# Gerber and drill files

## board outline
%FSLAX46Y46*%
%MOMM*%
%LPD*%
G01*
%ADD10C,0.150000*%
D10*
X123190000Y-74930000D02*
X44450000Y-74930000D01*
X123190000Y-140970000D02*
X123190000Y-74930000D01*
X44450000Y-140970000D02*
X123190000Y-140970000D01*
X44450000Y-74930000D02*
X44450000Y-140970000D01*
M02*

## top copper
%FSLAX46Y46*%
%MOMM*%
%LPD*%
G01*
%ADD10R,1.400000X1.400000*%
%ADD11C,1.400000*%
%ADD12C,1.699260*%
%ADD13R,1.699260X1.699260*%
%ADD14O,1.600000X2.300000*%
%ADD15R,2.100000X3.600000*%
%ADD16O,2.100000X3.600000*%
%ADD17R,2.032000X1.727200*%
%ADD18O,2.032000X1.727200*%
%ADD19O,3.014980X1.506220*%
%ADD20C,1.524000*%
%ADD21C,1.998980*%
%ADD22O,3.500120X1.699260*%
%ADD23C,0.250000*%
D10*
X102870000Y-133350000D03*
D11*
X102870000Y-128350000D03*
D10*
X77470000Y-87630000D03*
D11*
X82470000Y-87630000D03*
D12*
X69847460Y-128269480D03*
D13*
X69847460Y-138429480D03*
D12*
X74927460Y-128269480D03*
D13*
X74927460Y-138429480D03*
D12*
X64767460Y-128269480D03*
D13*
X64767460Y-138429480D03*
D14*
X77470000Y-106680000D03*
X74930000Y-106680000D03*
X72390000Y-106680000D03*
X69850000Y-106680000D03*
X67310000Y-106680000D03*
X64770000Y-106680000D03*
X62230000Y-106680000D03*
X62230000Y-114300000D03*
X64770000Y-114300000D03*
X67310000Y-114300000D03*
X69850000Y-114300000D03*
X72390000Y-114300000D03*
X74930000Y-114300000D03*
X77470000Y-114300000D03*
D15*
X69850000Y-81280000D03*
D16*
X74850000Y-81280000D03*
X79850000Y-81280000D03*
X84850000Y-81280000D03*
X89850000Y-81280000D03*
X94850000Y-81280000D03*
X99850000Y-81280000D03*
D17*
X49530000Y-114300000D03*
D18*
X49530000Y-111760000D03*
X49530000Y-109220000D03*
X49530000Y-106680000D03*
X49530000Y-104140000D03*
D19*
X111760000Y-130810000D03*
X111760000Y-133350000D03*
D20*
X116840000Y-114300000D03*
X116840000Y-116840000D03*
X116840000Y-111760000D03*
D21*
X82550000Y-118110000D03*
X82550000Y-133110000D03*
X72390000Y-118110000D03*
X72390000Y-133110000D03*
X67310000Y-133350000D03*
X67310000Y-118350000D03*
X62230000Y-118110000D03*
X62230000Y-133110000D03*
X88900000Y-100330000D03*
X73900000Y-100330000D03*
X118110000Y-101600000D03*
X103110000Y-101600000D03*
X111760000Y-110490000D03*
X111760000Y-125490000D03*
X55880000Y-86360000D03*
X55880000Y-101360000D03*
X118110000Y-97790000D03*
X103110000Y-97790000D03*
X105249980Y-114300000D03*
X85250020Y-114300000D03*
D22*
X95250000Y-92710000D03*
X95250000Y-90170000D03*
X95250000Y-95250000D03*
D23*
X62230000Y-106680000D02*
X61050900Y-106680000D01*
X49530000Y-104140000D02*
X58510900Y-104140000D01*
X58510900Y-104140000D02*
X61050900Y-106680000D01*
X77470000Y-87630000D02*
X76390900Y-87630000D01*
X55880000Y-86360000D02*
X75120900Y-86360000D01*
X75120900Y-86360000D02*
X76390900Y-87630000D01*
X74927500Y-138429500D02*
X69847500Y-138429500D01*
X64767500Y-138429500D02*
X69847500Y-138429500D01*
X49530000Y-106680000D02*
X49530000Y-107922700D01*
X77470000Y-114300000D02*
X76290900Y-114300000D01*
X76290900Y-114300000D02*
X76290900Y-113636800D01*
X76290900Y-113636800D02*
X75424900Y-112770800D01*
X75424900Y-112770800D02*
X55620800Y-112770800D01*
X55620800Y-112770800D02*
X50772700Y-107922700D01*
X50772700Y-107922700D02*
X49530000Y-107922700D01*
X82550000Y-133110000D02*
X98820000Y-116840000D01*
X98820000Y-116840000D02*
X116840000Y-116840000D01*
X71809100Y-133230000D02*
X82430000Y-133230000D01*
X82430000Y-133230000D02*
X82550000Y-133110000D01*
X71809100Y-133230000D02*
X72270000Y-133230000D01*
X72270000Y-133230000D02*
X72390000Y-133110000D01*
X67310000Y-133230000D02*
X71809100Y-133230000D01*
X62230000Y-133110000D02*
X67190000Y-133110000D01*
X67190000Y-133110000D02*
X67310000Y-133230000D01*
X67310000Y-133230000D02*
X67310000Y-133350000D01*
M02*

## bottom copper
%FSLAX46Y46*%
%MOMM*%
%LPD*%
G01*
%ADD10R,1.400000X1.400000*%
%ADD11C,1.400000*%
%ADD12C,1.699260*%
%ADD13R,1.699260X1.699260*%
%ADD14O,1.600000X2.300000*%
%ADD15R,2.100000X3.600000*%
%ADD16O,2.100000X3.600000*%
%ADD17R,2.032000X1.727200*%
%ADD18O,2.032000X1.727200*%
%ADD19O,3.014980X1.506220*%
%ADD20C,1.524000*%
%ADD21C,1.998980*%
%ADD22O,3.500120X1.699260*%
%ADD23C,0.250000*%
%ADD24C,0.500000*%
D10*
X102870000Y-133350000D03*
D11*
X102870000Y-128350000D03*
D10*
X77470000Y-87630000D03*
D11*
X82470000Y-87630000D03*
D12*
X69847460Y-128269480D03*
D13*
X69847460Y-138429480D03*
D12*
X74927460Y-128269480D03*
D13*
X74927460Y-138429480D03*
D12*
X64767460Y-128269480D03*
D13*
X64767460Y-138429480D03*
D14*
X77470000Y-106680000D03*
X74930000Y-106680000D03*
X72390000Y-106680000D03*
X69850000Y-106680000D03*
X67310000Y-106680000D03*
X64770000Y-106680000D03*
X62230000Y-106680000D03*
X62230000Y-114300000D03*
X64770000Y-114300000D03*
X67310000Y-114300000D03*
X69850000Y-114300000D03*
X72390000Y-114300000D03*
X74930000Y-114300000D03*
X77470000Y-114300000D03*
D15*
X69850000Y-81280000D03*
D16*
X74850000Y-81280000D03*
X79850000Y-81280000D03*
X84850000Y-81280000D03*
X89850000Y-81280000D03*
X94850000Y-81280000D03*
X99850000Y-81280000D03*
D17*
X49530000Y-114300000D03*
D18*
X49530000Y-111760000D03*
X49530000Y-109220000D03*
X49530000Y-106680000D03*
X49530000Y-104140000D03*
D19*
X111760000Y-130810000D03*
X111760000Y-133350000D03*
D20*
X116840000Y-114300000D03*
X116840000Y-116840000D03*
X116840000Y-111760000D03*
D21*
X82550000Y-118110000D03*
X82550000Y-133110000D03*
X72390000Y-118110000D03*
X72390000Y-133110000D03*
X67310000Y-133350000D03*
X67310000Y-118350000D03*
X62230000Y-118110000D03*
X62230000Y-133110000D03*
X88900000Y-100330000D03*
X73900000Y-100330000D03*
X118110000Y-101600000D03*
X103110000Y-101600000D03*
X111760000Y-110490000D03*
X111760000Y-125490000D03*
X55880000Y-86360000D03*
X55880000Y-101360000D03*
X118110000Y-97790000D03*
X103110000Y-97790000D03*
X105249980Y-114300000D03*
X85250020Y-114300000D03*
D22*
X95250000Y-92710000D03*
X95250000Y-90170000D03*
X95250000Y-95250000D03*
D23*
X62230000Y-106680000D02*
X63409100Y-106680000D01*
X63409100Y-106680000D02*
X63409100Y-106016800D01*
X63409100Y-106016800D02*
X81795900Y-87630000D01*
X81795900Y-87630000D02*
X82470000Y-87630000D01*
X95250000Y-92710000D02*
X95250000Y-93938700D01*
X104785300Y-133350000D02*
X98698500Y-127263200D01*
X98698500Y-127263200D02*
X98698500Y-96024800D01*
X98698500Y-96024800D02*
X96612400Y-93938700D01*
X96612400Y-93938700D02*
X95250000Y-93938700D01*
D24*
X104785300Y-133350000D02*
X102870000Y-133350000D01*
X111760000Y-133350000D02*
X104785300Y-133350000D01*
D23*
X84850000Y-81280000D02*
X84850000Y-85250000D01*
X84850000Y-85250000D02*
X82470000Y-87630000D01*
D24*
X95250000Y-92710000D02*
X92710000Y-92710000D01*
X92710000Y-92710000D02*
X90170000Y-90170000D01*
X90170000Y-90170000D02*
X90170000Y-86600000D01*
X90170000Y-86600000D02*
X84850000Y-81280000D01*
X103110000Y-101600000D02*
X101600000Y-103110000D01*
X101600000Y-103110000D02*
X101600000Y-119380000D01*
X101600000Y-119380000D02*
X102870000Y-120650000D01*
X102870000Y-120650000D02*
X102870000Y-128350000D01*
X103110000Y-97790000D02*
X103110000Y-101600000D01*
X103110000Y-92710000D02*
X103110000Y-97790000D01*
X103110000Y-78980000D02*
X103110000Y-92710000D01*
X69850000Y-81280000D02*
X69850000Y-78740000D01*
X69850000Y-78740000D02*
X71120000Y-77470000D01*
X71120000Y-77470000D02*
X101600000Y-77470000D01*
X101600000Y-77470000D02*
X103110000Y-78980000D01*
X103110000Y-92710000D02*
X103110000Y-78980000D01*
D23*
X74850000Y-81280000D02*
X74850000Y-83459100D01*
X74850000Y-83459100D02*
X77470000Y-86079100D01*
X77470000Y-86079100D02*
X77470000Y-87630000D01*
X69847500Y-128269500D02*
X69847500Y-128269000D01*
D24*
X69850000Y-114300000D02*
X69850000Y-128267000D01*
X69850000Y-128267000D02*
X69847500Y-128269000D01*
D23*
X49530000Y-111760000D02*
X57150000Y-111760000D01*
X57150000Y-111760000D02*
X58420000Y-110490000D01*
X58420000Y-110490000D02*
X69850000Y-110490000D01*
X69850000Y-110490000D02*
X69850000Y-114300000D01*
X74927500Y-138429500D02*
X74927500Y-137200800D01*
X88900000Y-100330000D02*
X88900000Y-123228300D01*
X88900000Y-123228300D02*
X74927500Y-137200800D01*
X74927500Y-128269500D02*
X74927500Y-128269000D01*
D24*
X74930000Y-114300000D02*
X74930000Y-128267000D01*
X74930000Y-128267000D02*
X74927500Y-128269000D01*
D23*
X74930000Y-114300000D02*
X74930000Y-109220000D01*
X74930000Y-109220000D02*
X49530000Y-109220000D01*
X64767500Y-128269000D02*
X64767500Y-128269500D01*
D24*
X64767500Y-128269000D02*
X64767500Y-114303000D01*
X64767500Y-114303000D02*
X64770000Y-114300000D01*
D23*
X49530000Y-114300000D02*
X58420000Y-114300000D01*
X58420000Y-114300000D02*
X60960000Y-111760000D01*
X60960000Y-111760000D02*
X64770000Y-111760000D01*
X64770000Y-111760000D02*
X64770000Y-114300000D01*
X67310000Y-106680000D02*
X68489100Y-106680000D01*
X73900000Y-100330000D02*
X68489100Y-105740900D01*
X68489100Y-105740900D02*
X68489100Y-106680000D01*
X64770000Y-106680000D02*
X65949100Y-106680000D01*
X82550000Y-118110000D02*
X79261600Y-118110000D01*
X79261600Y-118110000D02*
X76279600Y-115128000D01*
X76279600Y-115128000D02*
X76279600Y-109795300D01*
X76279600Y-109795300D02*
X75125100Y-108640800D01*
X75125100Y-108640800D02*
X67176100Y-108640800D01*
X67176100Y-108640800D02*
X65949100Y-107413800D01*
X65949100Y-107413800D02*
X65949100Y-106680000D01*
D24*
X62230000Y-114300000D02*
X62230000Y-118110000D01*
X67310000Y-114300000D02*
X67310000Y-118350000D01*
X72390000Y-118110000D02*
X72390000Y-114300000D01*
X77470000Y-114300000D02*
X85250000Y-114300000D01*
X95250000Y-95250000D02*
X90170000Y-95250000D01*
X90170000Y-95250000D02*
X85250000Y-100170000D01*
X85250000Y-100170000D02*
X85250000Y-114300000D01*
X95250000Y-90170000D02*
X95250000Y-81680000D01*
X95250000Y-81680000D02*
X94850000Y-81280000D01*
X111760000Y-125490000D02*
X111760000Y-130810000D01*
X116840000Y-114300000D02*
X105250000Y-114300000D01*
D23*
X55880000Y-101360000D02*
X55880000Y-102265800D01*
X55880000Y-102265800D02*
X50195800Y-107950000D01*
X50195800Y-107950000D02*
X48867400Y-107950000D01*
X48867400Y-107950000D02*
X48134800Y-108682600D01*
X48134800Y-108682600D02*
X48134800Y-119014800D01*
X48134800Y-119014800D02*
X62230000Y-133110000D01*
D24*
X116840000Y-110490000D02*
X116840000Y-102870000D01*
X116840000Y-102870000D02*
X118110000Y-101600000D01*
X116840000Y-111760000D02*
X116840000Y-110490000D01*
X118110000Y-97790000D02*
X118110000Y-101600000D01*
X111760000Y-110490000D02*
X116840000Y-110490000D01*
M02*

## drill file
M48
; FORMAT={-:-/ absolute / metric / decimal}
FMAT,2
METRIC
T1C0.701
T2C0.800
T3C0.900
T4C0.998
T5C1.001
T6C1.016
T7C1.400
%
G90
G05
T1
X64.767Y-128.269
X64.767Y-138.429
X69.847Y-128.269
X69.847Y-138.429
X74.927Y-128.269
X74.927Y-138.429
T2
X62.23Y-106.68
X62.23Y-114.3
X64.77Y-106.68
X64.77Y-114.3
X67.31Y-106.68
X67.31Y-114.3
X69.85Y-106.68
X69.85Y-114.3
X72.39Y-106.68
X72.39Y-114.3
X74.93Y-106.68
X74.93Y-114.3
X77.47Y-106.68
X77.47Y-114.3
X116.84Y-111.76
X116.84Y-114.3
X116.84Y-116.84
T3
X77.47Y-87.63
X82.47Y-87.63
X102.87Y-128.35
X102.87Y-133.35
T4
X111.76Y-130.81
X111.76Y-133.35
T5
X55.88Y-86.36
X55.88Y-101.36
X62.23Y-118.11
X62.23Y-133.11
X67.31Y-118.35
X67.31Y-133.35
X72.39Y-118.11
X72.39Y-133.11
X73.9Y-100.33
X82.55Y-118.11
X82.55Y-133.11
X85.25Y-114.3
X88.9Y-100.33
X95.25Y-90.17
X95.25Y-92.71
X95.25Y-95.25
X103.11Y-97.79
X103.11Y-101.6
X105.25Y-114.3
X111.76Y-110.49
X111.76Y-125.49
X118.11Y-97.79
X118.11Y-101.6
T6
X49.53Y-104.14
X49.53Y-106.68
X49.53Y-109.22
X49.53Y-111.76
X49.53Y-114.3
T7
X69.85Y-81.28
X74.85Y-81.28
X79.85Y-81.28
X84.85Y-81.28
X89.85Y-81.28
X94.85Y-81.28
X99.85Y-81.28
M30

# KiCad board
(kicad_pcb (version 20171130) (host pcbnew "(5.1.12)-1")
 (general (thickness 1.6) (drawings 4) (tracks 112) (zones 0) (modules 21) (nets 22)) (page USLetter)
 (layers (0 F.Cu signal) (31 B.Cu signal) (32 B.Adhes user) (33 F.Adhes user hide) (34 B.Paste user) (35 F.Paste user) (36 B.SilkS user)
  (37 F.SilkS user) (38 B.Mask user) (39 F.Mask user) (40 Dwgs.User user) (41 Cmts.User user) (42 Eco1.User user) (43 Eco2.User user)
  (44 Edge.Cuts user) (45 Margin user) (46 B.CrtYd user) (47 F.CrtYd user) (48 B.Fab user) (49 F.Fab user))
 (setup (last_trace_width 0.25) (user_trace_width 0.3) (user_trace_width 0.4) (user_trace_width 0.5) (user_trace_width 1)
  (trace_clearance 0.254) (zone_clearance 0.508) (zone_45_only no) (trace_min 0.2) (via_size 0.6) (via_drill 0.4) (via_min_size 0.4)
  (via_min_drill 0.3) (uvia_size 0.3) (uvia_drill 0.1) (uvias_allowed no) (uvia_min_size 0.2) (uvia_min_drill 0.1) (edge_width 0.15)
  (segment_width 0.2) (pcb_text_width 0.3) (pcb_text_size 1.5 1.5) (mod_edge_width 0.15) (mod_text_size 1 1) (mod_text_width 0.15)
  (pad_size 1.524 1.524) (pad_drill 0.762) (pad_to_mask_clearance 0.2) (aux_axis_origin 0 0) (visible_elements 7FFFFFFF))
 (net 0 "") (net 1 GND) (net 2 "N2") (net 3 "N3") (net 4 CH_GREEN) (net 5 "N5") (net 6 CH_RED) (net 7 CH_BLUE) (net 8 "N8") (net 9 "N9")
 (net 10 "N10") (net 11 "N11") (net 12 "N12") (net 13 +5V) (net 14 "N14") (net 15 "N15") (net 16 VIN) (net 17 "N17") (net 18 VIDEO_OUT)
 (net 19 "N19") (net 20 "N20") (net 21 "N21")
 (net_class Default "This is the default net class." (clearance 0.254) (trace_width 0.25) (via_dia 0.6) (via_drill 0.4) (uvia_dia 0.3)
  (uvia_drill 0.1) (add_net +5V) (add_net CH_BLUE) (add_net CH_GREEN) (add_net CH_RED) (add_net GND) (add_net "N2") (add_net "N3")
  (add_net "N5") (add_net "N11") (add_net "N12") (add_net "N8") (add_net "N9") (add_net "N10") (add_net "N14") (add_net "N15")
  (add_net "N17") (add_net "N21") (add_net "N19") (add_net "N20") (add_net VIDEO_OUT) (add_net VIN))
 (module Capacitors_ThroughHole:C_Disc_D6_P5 (layer F.Cu) (at 102.87 133.35 90)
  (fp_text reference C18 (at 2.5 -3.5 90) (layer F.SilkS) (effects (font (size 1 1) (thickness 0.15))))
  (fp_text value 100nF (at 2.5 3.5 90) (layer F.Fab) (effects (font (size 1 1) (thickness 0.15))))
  (pad 1 thru_hole rect (at 0 0 90) (size 1.4 1.4) (drill 0.9) (layers *.Cu *.Mask F.SilkS) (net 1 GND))
  (pad 2 thru_hole circle (at 5 0 90) (size 1.4 1.4) (drill 0.9) (layers *.Cu *.Mask F.SilkS) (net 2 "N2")))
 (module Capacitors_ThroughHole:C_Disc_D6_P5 (layer F.Cu) (at 77.47 87.63)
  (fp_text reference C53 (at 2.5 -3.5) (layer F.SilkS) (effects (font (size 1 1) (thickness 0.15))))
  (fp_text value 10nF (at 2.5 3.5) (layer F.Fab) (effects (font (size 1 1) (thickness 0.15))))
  (pad 1 thru_hole rect (at 0 0) (size 1.4 1.4) (drill 0.9) (layers *.Cu *.Mask F.SilkS) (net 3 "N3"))
  (pad 2 thru_hole circle (at 5 0) (size 1.4 1.4) (drill 0.9) (layers *.Cu *.Mask F.SilkS) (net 1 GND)))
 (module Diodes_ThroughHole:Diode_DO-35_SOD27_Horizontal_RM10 (layer F.Cu) (at 69.85 138.43 90)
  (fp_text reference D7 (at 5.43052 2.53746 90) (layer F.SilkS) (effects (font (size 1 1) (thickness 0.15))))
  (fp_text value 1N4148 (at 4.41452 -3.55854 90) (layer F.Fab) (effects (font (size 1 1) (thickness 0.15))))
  (pad 2 thru_hole circle (at 10.16052 -0.00254 270) (size 1.69926 1.69926) (drill 0.70104) (layers *.Cu *.Mask F.SilkS) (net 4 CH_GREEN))
  (pad 1 thru_hole rect (at 0.00052 -0.00254 270) (size 1.69926 1.69926) (drill 0.70104) (layers *.Cu *.Mask F.SilkS) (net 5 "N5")))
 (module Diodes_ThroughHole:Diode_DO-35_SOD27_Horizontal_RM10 (layer F.Cu) (at 74.93 138.43 90)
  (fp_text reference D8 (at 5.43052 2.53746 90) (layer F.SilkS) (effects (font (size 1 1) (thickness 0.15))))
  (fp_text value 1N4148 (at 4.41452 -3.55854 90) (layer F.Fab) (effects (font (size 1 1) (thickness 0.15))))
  (pad 2 thru_hole circle (at 10.16052 -0.00254 270) (size 1.69926 1.69926) (drill 0.70104) (layers *.Cu *.Mask F.SilkS) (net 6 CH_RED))
  (pad 1 thru_hole rect (at 0.00052 -0.00254 270) (size 1.69926 1.69926) (drill 0.70104) (layers *.Cu *.Mask F.SilkS) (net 5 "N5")))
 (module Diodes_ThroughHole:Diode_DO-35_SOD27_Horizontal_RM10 (layer F.Cu) (at 64.77 138.43 90)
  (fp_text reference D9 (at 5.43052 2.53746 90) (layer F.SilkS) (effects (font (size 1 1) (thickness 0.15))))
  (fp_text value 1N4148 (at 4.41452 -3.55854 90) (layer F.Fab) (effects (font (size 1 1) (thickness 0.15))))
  (pad 2 thru_hole circle (at 10.16052 -0.00254 270) (size 1.69926 1.69926) (drill 0.70104) (layers *.Cu *.Mask F.SilkS) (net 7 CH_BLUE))
  (pad 1 thru_hole rect (at 0.00052 -0.00254 270) (size 1.69926 1.69926) (drill 0.70104) (layers *.Cu *.Mask F.SilkS) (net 5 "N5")))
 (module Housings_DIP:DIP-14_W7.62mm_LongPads (layer F.Cu) (at 77.47 106.68 270)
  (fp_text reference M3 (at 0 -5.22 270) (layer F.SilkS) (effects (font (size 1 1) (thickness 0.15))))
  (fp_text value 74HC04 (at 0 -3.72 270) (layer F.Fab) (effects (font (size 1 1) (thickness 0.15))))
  (pad 1 thru_hole oval (at 0 0 270) (size 2.3 1.6) (drill 0.8) (layers *.Cu *.Mask F.SilkS))
  (pad 2 thru_hole oval (at 0 2.54 270) (size 2.3 1.6) (drill 0.8) (layers *.Cu *.Mask F.SilkS))
  (pad 3 thru_hole oval (at 0 5.08 270) (size 2.3 1.6) (drill 0.8) (layers *.Cu *.Mask F.SilkS))
  (pad 4 thru_hole oval (at 0 7.62 270) (size 2.3 1.6) (drill 0.8) (layers *.Cu *.Mask F.SilkS))
  (pad 5 thru_hole oval (at 0 10.16 270) (size 2.3 1.6) (drill 0.8) (layers *.Cu *.Mask F.SilkS) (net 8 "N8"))
  (pad 6 thru_hole oval (at 0 12.7 270) (size 2.3 1.6) (drill 0.8) (layers *.Cu *.Mask F.SilkS) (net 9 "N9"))
  (pad 7 thru_hole oval (at 0 15.24 270) (size 2.3 1.6) (drill 0.8) (layers *.Cu *.Mask F.SilkS) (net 1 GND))
  (pad 8 thru_hole oval (at 7.62 15.24 270) (size 2.3 1.6) (drill 0.8) (layers *.Cu *.Mask F.SilkS) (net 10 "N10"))
  (pad 9 thru_hole oval (at 7.62 12.7 270) (size 2.3 1.6) (drill 0.8) (layers *.Cu *.Mask F.SilkS) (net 7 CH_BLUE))
  (pad 10 thru_hole oval (at 7.62 10.16 270) (size 2.3 1.6) (drill 0.8) (layers *.Cu *.Mask F.SilkS) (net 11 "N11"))
  (pad 11 thru_hole oval (at 7.62 7.62 270) (size 2.3 1.6) (drill 0.8) (layers *.Cu *.Mask F.SilkS) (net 4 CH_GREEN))
  (pad 12 thru_hole oval (at 7.62 5.08 270) (size 2.3 1.6) (drill 0.8) (layers *.Cu *.Mask F.SilkS) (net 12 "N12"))
  (pad 13 thru_hole oval (at 7.62 2.54 270) (size 2.3 1.6) (drill 0.8) (layers *.Cu *.Mask F.SilkS) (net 6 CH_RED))
  (pad 14 thru_hole oval (at 7.62 0 270) (size 2.3 1.6) (drill 0.8) (layers *.Cu *.Mask F.SilkS) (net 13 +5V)))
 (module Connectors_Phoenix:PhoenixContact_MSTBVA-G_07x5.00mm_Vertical (layer F.Cu) (at 69.85 81.28)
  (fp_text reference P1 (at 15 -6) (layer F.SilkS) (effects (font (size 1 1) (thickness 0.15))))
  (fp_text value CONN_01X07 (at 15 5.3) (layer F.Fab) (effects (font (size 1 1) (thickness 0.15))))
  (pad 1 thru_hole rect (at 0 0) (size 2.1 3.6) (drill 1.4) (layers *.Cu *.Mask) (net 2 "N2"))
  (pad 2 thru_hole oval (at 5 0) (size 2.1 3.6) (drill 1.4) (layers *.Cu *.Mask) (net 3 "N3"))
  (pad 3 thru_hole oval (at 10 0) (size 2.1 3.6) (drill 1.4) (layers *.Cu *.Mask) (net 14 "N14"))
  (pad 4 thru_hole oval (at 15 0) (size 2.1 3.6) (drill 1.4) (layers *.Cu *.Mask) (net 1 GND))
  (pad 5 thru_hole oval (at 20 0) (size 2.1 3.6) (drill 1.4) (layers *.Cu *.Mask) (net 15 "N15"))
  (pad 6 thru_hole oval (at 25 0) (size 2.1 3.6) (drill 1.4) (layers *.Cu *.Mask) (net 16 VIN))
  (pad 7 thru_hole oval (at 30 0) (size 2.1 3.6) (drill 1.4) (layers *.Cu *.Mask) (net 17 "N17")))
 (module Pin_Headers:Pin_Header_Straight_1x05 (layer B.Cu) (at 49.53 114.3)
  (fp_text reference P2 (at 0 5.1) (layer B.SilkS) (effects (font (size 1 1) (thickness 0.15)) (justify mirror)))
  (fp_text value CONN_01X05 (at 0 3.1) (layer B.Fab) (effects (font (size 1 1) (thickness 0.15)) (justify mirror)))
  (pad 1 thru_hole rect (at 0 0) (size 2.032 1.7272) (drill 1.016) (layers *.Cu *.Mask B.SilkS) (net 7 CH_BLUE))
  (pad 2 thru_hole oval (at 0 -2.54) (size 2.032 1.7272) (drill 1.016) (layers *.Cu *.Mask B.SilkS) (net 4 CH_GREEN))
  (pad 3 thru_hole oval (at 0 -5.08) (size 2.032 1.7272) (drill 1.016) (layers *.Cu *.Mask B.SilkS) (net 6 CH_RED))
  (pad 4 thru_hole oval (at 0 -7.62) (size 2.032 1.7272) (drill 1.016) (layers *.Cu *.Mask B.SilkS) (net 13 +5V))
  (pad 5 thru_hole oval (at 0 -10.16) (size 2.032 1.7272) (drill 1.016) (layers *.Cu *.Mask B.SilkS) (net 1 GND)))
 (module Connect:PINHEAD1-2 (layer F.Cu) (at 111.76 132.08 270)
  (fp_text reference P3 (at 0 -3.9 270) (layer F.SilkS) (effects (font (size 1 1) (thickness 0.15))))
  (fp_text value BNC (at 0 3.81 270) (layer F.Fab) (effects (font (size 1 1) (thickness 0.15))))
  (pad 1 thru_hole oval (at -1.27 0 270) (size 1.50622 3.01498) (drill 0.99822) (layers *.Cu *.Mask) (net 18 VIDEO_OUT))
  (pad 2 thru_hole oval (at 1.27 0 270) (size 1.50622 3.01498) (drill 0.99822) (layers *.Cu *.Mask) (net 1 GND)))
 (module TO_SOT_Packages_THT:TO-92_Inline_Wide (layer F.Cu) (at 116.84 111.76 270)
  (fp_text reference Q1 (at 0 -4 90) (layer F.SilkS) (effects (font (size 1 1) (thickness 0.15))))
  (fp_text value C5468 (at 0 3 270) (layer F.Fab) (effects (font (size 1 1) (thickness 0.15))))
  (pad 2 thru_hole circle (at 2.54 0) (size 1.524 1.524) (drill 0.8) (layers *.Cu *.Mask F.SilkS) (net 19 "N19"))
  (pad 3 thru_hole circle (at 5.08 0) (size 1.524 1.524) (drill 0.8) (layers *.Cu *.Mask F.SilkS) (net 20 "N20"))
  (pad 1 thru_hole circle (at 0 0) (size 1.524 1.524) (drill 0.8) (layers *.Cu *.Mask F.SilkS) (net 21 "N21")))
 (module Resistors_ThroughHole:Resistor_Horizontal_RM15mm (layer F.Cu) (at 82.55 118.11 270)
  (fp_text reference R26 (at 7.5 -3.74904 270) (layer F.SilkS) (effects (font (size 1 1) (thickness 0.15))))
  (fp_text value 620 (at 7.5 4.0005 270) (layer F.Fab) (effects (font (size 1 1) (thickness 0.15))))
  (pad 1 thru_hole circle (at 0 0 270) (size 1.99898 1.99898) (drill 1.00076) (layers *.Cu *.SilkS *.Mask) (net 9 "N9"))
  (pad 2 thru_hole circle (at 15 0 270) (size 1.99898 1.99898) (drill 1.00076) (layers *.Cu *.SilkS *.Mask) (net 20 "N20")))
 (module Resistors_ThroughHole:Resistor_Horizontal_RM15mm (layer F.Cu) (at 72.39 118.11 270)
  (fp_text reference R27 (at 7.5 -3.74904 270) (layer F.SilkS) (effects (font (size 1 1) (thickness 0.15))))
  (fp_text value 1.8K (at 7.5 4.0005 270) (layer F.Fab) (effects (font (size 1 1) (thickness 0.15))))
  (pad 1 thru_hole circle (at 0 0 270) (size 1.99898 1.99898) (drill 1.00076) (layers *.Cu *.SilkS *.Mask) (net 12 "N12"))
  (pad 2 thru_hole circle (at 15 0 270) (size 1.99898 1.99898) (drill 1.00076) (layers *.Cu *.SilkS *.Mask) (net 20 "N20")))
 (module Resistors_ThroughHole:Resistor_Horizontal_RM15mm (layer F.Cu) (at 67.31 133.35 90)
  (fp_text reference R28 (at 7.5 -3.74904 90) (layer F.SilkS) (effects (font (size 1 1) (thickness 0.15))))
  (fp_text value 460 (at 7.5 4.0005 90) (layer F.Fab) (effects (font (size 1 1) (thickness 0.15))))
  (pad 1 thru_hole circle (at 0 0 90) (size 1.99898 1.99898) (drill 1.00076) (layers *.Cu *.SilkS *.Mask) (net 20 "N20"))
  (pad 2 thru_hole circle (at 15 0 90) (size 1.99898 1.99898) (drill 1.00076) (layers *.Cu *.SilkS *.Mask) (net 11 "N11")))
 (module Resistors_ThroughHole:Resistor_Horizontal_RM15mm (layer F.Cu) (at 62.23 118.11 270)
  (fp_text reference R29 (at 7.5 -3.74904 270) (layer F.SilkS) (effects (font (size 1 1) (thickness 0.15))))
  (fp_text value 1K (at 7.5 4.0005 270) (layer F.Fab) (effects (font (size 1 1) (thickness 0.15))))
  (pad 1 thru_hole circle (at 0 0 270) (size 1.99898 1.99898) (drill 1.00076) (layers *.Cu *.SilkS *.Mask) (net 10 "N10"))
  (pad 2 thru_hole circle (at 15 0 270) (size 1.99898 1.99898) (drill 1.00076) (layers *.Cu *.SilkS *.Mask) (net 20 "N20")))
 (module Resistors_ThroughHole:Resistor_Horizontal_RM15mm (layer F.Cu) (at 88.9 100.33 180)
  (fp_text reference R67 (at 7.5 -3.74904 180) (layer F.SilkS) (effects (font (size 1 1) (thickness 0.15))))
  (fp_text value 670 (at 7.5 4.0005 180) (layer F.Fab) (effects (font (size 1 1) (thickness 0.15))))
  (pad 1 thru_hole circle (at 0 0 180) (size 1.99898 1.99898) (drill 1.00076) (layers *.Cu *.SilkS *.Mask) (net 5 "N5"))
  (pad 2 thru_hole circle (at 15 0 180) (size 1.99898 1.99898) (drill 1.00076) (layers *.Cu *.SilkS *.Mask) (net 8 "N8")))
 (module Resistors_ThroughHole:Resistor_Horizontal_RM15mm (layer F.Cu) (at 118.11 101.6 180)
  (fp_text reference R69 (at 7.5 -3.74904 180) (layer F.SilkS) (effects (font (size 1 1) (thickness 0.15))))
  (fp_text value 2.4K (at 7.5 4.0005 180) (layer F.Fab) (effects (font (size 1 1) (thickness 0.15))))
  (pad 1 thru_hole circle (at 0 0 180) (size 1.99898 1.99898) (drill 1.00076) (layers *.Cu *.SilkS *.Mask) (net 21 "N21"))
  (pad 2 thru_hole circle (at 15 0 180) (size 1.99898 1.99898) (drill 1.00076) (layers *.Cu *.SilkS *.Mask) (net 2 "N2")))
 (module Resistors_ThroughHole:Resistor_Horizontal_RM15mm (layer F.Cu) (at 111.76 110.49 270)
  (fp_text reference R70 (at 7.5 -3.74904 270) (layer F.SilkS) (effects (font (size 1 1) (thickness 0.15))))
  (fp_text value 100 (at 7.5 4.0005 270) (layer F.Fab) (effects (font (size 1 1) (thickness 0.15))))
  (pad 1 thru_hole circle (at 0 0 270) (size 1.99898 1.99898) (drill 1.00076) (layers *.Cu *.SilkS *.Mask) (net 21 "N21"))
  (pad 2 thru_hole circle (at 15 0 270) (size 1.99898 1.99898) (drill 1.00076) (layers *.Cu *.SilkS *.Mask) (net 18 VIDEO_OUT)))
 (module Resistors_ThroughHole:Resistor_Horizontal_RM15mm (layer F.Cu) (at 55.88 86.36 270)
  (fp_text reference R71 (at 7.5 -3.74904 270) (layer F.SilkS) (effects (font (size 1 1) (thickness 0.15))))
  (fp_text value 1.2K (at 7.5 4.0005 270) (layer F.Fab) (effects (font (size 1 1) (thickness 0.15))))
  (pad 1 thru_hole circle (at 0 0 270) (size 1.99898 1.99898) (drill 1.00076) (layers *.Cu *.SilkS *.Mask) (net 3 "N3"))
  (pad 2 thru_hole circle (at 15 0 270) (size 1.99898 1.99898) (drill 1.00076) (layers *.Cu *.SilkS *.Mask) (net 20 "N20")))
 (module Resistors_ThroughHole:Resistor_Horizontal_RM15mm (layer F.Cu) (at 118.11 97.79 180)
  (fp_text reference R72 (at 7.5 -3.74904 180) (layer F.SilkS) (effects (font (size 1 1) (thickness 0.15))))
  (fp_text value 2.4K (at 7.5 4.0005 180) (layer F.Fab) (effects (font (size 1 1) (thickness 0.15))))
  (pad 1 thru_hole circle (at 0 0 180) (size 1.99898 1.99898) (drill 1.00076) (layers *.Cu *.SilkS *.Mask) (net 21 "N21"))
  (pad 2 thru_hole circle (at 15 0 180) (size 1.99898 1.99898) (drill 1.00076) (layers *.Cu *.SilkS *.Mask) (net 2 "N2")))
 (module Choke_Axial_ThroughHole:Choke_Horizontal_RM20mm (layer F.Cu) (at 95.25 114.3 180)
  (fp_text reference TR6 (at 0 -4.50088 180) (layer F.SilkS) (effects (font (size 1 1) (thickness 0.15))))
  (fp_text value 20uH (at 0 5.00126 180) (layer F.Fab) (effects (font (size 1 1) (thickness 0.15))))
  (pad 1 thru_hole circle (at -9.99998 0 180) (size 1.99898 1.99898) (drill 1.00076) (layers *.Cu *.Mask F.SilkS) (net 19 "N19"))
  (pad 2 thru_hole circle (at 9.99998 0 180) (size 1.99898 1.99898) (drill 1.00076) (layers *.Cu *.Mask F.SilkS) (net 13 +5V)))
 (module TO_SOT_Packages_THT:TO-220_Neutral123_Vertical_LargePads (layer F.Cu) (at 95.25 92.71 270)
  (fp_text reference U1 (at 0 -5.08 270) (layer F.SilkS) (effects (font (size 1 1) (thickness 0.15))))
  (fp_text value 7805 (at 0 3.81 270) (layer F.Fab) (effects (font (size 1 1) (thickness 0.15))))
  (pad 2 thru_hole oval (at 0 0) (size 3.50012 1.69926) (drill 1.00076) (layers *.Cu *.Mask F.SilkS) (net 1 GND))
  (pad 1 thru_hole oval (at -2.54 0) (size 3.50012 1.69926) (drill 1.00076) (layers *.Cu *.Mask F.SilkS) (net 16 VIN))
  (pad 3 thru_hole oval (at 2.54 0) (size 3.50012 1.69926) (drill 1.00076) (layers *.Cu *.Mask F.SilkS) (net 13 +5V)))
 (gr_line (start 123.19 74.93) (end 44.45 74.93) (angle 90) (layer Edge.Cuts) (width 0.15))
 (gr_line (start 123.19 140.97) (end 123.19 74.93) (angle 90) (layer Edge.Cuts) (width 0.15))
 (gr_line (start 44.45 140.97) (end 123.19 140.97) (angle 90) (layer Edge.Cuts) (width 0.15))
 (gr_line (start 44.45 74.93) (end 44.45 140.97) (angle 90) (layer Edge.Cuts) (width 0.15))
 (segment (start 62.23 106.68) (end 63.4091 106.68) (width 0.25) (layer B.Cu) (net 1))
 (segment (start 63.4091 106.68) (end 63.4091 106.0168) (width 0.25) (layer B.Cu) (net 1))
 (segment (start 63.4091 106.0168) (end 81.7959 87.63) (width 0.25) (layer B.Cu) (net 1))
 (segment (start 81.7959 87.63) (end 82.47 87.63) (width 0.25) (layer B.Cu) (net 1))
 (segment (start 62.23 106.68) (end 61.0509 106.68) (width 0.25) (layer F.Cu) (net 1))
 (segment (start 49.53 104.14) (end 58.5109 104.14) (width 0.25) (layer F.Cu) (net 1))
 (segment (start 58.5109 104.14) (end 61.0509 106.68) (width 0.25) (layer F.Cu) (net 1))
 (segment (start 95.25 92.71) (end 95.25 93.9387) (width 0.25) (layer B.Cu) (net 1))
 (segment (start 104.7853 133.35) (end 98.6985 127.2632) (width 0.25) (layer B.Cu) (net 1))
 (segment (start 98.6985 127.2632) (end 98.6985 96.0248) (width 0.25) (layer B.Cu) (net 1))
 (segment (start 98.6985 96.0248) (end 96.6124 93.9387) (width 0.25) (layer B.Cu) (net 1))
 (segment (start 96.6124 93.9387) (end 95.25 93.9387) (width 0.25) (layer B.Cu) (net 1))
 (segment (start 104.7853 133.35) (end 102.87 133.35) (width 0.5) (layer B.Cu) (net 1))
 (segment (start 111.76 133.35) (end 104.7853 133.35) (width 0.5) (layer B.Cu) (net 1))
 (segment (start 84.85 81.28) (end 84.85 85.25) (width 0.25) (layer B.Cu) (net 1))
 (segment (start 84.85 85.25) (end 82.47 87.63) (width 0.25) (layer B.Cu) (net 1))
 (segment (start 95.25 92.71) (end 92.71 92.71) (width 0.5) (layer B.Cu) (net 1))
 (segment (start 92.71 92.71) (end 90.17 90.17) (width 0.5) (layer B.Cu) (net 1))
 (segment (start 90.17 90.17) (end 90.17 86.6) (width 0.5) (layer B.Cu) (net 1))
 (segment (start 90.17 86.6) (end 84.85 81.28) (width 0.5) (layer B.Cu) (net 1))
 (segment (start 103.11 101.6) (end 101.6 103.11) (width 0.5) (layer B.Cu) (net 2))
 (segment (start 101.6 103.11) (end 101.6 119.38) (width 0.5) (layer B.Cu) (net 2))
 (segment (start 101.6 119.38) (end 102.87 120.65) (width 0.5) (layer B.Cu) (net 2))
 (segment (start 102.87 120.65) (end 102.87 128.35) (width 0.5) (layer B.Cu) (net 2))
 (segment (start 103.11 97.79) (end 103.11 101.6) (width 0.5) (layer B.Cu) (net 2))
 (segment (start 103.11 92.71) (end 103.11 97.79) (width 0.5) (layer B.Cu) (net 2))
 (segment (start 103.11 78.98) (end 103.11 92.71) (width 0.5) (layer B.Cu) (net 2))
 (segment (start 69.85 81.28) (end 69.85 78.74) (width 0.5) (layer B.Cu) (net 2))
 (segment (start 69.85 78.74) (end 71.12 77.47) (width 0.5) (layer B.Cu) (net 2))
 (segment (start 71.12 77.47) (end 101.6 77.47) (width 0.5) (layer B.Cu) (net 2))
 (segment (start 101.6 77.47) (end 103.11 78.98) (width 0.5) (layer B.Cu) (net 2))
 (segment (start 103.11 92.71) (end 103.11 78.98) (width 0.5) (layer B.Cu) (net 2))
 (segment (start 74.85 81.28) (end 74.85 83.4591) (width 0.25) (layer B.Cu) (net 3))
 (segment (start 74.85 83.4591) (end 77.47 86.0791) (width 0.25) (layer B.Cu) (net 3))
 (segment (start 77.47 86.0791) (end 77.47 87.63) (width 0.25) (layer B.Cu) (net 3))
 (segment (start 77.47 87.63) (end 76.3909 87.63) (width 0.25) (layer F.Cu) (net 3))
 (segment (start 55.88 86.36) (end 75.1209 86.36) (width 0.25) (layer F.Cu) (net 3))
 (segment (start 75.1209 86.36) (end 76.3909 87.63) (width 0.25) (layer F.Cu) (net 3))
 (segment (start 69.8475 128.2695) (end 69.8475 128.269) (width 0.25) (layer B.Cu) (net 4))
 (segment (start 69.85 114.3) (end 69.85 128.267) (width 0.5) (layer B.Cu) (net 4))
 (segment (start 69.85 128.267) (end 69.8475 128.269) (width 0.5) (layer B.Cu) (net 4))
 (segment (start 49.53 111.76) (end 57.15 111.76) (width 0.25) (layer B.Cu) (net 4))
 (segment (start 57.15 111.76) (end 58.42 110.49) (width 0.25) (layer B.Cu) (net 4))
 (segment (start 58.42 110.49) (end 69.85 110.49) (width 0.25) (layer B.Cu) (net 4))
 (segment (start 69.85 110.49) (end 69.85 114.3) (width 0.25) (layer B.Cu) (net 4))
 (segment (start 74.9275 138.4295) (end 69.8475 138.4295) (width 0.25) (layer F.Cu) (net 5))
 (segment (start 64.7675 138.4295) (end 69.8475 138.4295) (width 0.25) (layer F.Cu) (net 5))
 (segment (start 74.9275 138.4295) (end 74.9275 137.2008) (width 0.25) (layer B.Cu) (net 5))
 (segment (start 88.9 100.33) (end 88.9 123.2283) (width 0.25) (layer B.Cu) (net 5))
 (segment (start 88.9 123.2283) (end 74.9275 137.2008) (width 0.25) (layer B.Cu) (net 5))
 (segment (start 74.9275 128.2695) (end 74.9275 128.269) (width 0.25) (layer B.Cu) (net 6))
 (segment (start 74.93 114.3) (end 74.93 128.267) (width 0.5) (layer B.Cu) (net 6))
 (segment (start 74.93 128.267) (end 74.9275 128.269) (width 0.5) (layer B.Cu) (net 6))
 (segment (start 74.93 114.3) (end 74.93 109.22) (width 0.25) (layer B.Cu) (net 6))
 (segment (start 74.93 109.22) (end 49.53 109.22) (width 0.25) (layer B.Cu) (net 6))
 (segment (start 64.7675 128.269) (end 64.7675 128.2695) (width 0.25) (layer B.Cu) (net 7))
 (segment (start 64.7675 128.269) (end 64.7675 114.303) (width 0.5) (layer B.Cu) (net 7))
 (segment (start 64.7675 114.303) (end 64.77 114.3) (width 0.5) (layer B.Cu) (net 7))
 (segment (start 49.53 114.3) (end 58.42 114.3) (width 0.25) (layer B.Cu) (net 7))
 (segment (start 58.42 114.3) (end 60.96 111.76) (width 0.25) (layer B.Cu) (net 7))
 (segment (start 60.96 111.76) (end 64.77 111.76) (width 0.25) (layer B.Cu) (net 7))
 (segment (start 64.77 111.76) (end 64.77 114.3) (width 0.25) (layer B.Cu) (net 7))
 (segment (start 67.31 106.68) (end 68.4891 106.68) (width 0.25) (layer B.Cu) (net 8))
 (segment (start 73.9 100.33) (end 68.4891 105.7409) (width 0.25) (layer B.Cu) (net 8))
 (segment (start 68.4891 105.7409) (end 68.4891 106.68) (width 0.25) (layer B.Cu) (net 8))
 (segment (start 64.77 106.68) (end 65.9491 106.68) (width 0.25) (layer B.Cu) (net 9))
 (segment (start 82.55 118.11) (end 79.2616 118.11) (width 0.25) (layer B.Cu) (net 9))
 (segment (start 79.2616 118.11) (end 76.2796 115.128) (width 0.25) (layer B.Cu) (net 9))
 (segment (start 76.2796 115.128) (end 76.2796 109.7953) (width 0.25) (layer B.Cu) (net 9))
 (segment (start 76.2796 109.7953) (end 75.1251 108.6408) (width 0.25) (layer B.Cu) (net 9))
 (segment (start 75.1251 108.6408) (end 67.1761 108.6408) (width 0.25) (layer B.Cu) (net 9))
 (segment (start 67.1761 108.6408) (end 65.9491 107.4138) (width 0.25) (layer B.Cu) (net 9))
 (segment (start 65.9491 107.4138) (end 65.9491 106.68) (width 0.25) (layer B.Cu) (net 9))
 (segment (start 62.23 114.3) (end 62.23 118.11) (width 0.5) (layer B.Cu) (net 10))
 (segment (start 67.31 114.3) (end 67.31 118.35) (width 0.5) (layer B.Cu) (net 11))
 (segment (start 72.39 118.11) (end 72.39 114.3) (width 0.5) (layer B.Cu) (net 12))
 (segment (start 49.53 106.68) (end 49.53 107.9227) (width 0.25) (layer F.Cu) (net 13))
 (segment (start 77.47 114.3) (end 76.2909 114.3) (width 0.25) (layer F.Cu) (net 13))
 (segment (start 76.2909 114.3) (end 76.2909 113.6368) (width 0.25) (layer F.Cu) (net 13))
 (segment (start 76.2909 113.6368) (end 75.4249 112.7708) (width 0.25) (layer F.Cu) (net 13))
 (segment (start 75.4249 112.7708) (end 55.6208 112.7708) (width 0.25) (layer F.Cu) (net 13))
 (segment (start 55.6208 112.7708) (end 50.7727 107.9227) (width 0.25) (layer F.Cu) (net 13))
 (segment (start 50.7727 107.9227) (end 49.53 107.9227) (width 0.25) (layer F.Cu) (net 13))
 (segment (start 77.47 114.3) (end 85.25 114.3) (width 0.5) (layer B.Cu) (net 13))
 (segment (start 95.25 95.25) (end 90.17 95.25) (width 0.5) (layer B.Cu) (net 13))
 (segment (start 90.17 95.25) (end 85.25 100.17) (width 0.5) (layer B.Cu) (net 13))
 (segment (start 85.25 100.17) (end 85.25 114.3) (width 0.5) (layer B.Cu) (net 13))
 (segment (start 95.25 90.17) (end 95.25 81.68) (width 0.5) (layer B.Cu) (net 16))
 (segment (start 95.25 81.68) (end 94.85 81.28) (width 0.5) (layer B.Cu) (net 16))
 (segment (start 111.76 125.49) (end 111.76 130.81) (width 0.5) (layer B.Cu) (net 18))
 (segment (start 116.84 114.3) (end 105.25 114.3) (width 0.5) (layer B.Cu) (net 19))
 (segment (start 82.55 133.11) (end 98.82 116.84) (width 0.25) (layer F.Cu) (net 20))
 (segment (start 98.82 116.84) (end 116.84 116.84) (width 0.25) (layer F.Cu) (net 20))
 (segment (start 71.8091 133.23) (end 82.43 133.23) (width 0.25) (layer F.Cu) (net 20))
 (segment (start 82.43 133.23) (end 82.55 133.11) (width 0.25) (layer F.Cu) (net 20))
 (segment (start 71.8091 133.23) (end 72.27 133.23) (width 0.25) (layer F.Cu) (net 20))
 (segment (start 72.27 133.23) (end 72.39 133.11) (width 0.25) (layer F.Cu) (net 20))
 (segment (start 67.31 133.23) (end 71.8091 133.23) (width 0.25) (layer F.Cu) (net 20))
 (segment (start 62.23 133.11) (end 67.19 133.11) (width 0.25) (layer F.Cu) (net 20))
 (segment (start 67.19 133.11) (end 67.31 133.23) (width 0.25) (layer F.Cu) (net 20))
 (segment (start 67.31 133.23) (end 67.31 133.35) (width 0.25) (layer F.Cu) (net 20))
 (segment (start 55.88 101.36) (end 55.88 102.2658) (width 0.25) (layer B.Cu) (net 20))
 (segment (start 55.88 102.2658) (end 50.1958 107.95) (width 0.25) (layer B.Cu) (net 20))
 (segment (start 50.1958 107.95) (end 48.8674 107.95) (width 0.25) (layer B.Cu) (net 20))
 (segment (start 48.8674 107.95) (end 48.1348 108.6826) (width 0.25) (layer B.Cu) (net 20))
 (segment (start 48.1348 108.6826) (end 48.1348 119.0148) (width 0.25) (layer B.Cu) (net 20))
 (segment (start 48.1348 119.0148) (end 62.23 133.11) (width 0.25) (layer B.Cu) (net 20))
 (segment (start 116.84 110.49) (end 116.84 102.87) (width 0.5) (layer B.Cu) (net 21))
 (segment (start 116.84 102.87) (end 118.11 101.6) (width 0.5) (layer B.Cu) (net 21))
 (segment (start 116.84 111.76) (end 116.84 110.49) (width 0.5) (layer B.Cu) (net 21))
 (segment (start 118.11 97.79) (end 118.11 101.6) (width 0.5) (layer B.Cu) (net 21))
 (segment (start 111.76 110.49) (end 116.84 110.49) (width 0.5) (layer B.Cu) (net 21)))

